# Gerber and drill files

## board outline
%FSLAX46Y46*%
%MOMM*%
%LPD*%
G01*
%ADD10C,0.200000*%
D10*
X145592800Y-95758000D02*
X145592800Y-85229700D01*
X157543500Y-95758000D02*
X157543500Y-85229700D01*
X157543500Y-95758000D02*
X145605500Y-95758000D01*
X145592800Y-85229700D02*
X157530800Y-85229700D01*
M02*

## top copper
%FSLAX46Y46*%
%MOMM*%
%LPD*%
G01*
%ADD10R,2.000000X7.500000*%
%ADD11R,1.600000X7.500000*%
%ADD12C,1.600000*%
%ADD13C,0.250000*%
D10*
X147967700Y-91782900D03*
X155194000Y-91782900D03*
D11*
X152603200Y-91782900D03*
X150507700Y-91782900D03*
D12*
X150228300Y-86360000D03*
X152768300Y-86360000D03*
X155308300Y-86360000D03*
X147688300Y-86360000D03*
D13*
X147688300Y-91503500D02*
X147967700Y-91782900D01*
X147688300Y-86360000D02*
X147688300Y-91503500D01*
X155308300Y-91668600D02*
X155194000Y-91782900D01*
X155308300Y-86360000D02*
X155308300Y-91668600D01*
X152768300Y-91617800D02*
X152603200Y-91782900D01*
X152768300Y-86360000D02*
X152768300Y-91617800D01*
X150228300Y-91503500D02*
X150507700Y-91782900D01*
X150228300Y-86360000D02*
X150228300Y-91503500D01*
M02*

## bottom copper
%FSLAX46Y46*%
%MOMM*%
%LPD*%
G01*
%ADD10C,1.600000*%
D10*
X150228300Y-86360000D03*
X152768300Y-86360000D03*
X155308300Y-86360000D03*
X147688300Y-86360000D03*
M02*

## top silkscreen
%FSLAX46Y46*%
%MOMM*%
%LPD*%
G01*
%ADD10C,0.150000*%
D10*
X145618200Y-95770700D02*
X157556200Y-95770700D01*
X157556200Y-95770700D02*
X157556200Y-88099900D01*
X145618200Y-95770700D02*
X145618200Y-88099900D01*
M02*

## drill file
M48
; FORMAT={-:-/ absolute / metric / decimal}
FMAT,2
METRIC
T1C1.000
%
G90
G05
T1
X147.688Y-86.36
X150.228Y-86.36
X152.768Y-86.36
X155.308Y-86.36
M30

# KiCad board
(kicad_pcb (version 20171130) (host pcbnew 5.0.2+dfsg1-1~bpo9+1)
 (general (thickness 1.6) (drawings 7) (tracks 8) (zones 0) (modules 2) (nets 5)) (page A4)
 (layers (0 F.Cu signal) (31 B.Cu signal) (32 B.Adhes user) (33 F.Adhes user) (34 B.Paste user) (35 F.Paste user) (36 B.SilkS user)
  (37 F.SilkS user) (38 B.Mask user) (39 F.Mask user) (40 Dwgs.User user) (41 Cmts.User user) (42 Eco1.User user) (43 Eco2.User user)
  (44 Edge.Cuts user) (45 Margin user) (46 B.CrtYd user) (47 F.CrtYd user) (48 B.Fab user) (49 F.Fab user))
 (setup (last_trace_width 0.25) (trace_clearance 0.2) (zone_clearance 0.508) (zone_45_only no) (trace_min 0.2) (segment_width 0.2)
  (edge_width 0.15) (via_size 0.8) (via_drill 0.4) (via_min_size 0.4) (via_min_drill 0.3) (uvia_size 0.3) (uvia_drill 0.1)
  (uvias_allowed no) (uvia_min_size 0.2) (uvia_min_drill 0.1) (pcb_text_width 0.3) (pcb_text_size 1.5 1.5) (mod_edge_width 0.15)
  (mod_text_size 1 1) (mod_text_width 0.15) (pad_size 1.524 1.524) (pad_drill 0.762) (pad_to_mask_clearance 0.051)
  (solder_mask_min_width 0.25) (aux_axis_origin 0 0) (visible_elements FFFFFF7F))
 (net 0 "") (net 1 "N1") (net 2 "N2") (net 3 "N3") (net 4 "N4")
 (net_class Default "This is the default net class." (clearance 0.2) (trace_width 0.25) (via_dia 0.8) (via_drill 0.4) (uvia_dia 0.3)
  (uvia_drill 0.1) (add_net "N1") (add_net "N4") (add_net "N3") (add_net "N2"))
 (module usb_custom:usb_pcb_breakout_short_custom (layer F.Cu) (at 151.5237 95.7707)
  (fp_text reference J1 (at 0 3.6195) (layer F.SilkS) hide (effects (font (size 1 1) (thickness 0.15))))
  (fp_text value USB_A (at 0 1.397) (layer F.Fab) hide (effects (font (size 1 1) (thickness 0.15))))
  (fp_line (start -5.9055 0) (end 6.0325 0) (layer F.SilkS) (width 0.15))
  (fp_line (start 6.0325 0) (end 6.0325 -7.6708) (layer F.SilkS) (width 0.15))
  (fp_line (start -5.9055 0) (end -5.9055 -7.6708) (layer F.SilkS) (width 0.15))
  (pad 1 smd rect (at -3.556 -3.9878) (size 2 7.5) (layers F.Cu F.Paste F.Mask) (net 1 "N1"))
  (pad 4 smd rect (at 3.6703 -3.9878) (size 2 7.5) (layers F.Cu F.Paste F.Mask) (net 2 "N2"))
  (pad 3 smd rect (at 1.0795 -3.9878) (size 1.6 7.5) (layers F.Cu F.Paste F.Mask) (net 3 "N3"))
  (pad 2 smd rect (at -1.016 -3.9878) (size 1.6 7.5) (layers F.Cu F.Paste F.Mask) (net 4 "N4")))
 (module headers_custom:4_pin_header (layer F.Cu) (at 151.4983 86.36)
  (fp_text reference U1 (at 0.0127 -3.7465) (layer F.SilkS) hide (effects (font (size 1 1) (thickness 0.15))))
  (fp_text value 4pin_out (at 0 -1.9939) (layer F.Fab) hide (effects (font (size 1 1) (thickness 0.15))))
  (pad 2 thru_hole circle (at -1.27 0) (size 1.6 1.6) (drill 1) (layers *.Cu *.Mask) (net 4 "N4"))
  (pad 3 thru_hole circle (at 1.27 0) (size 1.6 1.6) (drill 1) (layers *.Cu *.Mask) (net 3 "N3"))
  (pad 4 thru_hole circle (at 3.81 0) (size 1.6 1.6) (drill 1) (layers *.Cu *.Mask) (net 2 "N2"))
  (pad 1 thru_hole circle (at -3.81 0) (size 1.6 1.6) (drill 1) (layers *.Cu *.Mask) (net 1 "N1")))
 (gr_line (start 145.5928 95.758) (end 145.5928 85.2297) (layer Edge.Cuts) (width 0.2))
 (gr_line (start 157.5435 95.758) (end 157.5435 85.2297) (layer Edge.Cuts) (width 0.2))
 (gr_line (start 157.5435 95.758) (end 145.6055 95.758) (layer Edge.Cuts) (width 0.2))
 (gr_line (start 145.5928 85.2297) (end 157.5308 85.2297) (layer Edge.Cuts) (width 0.2))
 (segment (start 147.6883 91.5035) (end 147.9677 91.7829) (width 0.25) (layer F.Cu) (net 1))
 (segment (start 147.6883 86.36) (end 147.6883 91.5035) (width 0.25) (layer F.Cu) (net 1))
 (segment (start 155.3083 91.6686) (end 155.194 91.7829) (width 0.25) (layer F.Cu) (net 2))
 (segment (start 155.3083 86.36) (end 155.3083 91.6686) (width 0.25) (layer F.Cu) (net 2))
 (segment (start 152.7683 91.6178) (end 152.6032 91.7829) (width 0.25) (layer F.Cu) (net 3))
 (segment (start 152.7683 86.36) (end 152.7683 91.6178) (width 0.25) (layer F.Cu) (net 3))
 (segment (start 150.2283 91.5035) (end 150.5077 91.7829) (width 0.25) (layer F.Cu) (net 4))
 (segment (start 150.2283 86.36) (end 150.2283 91.5035) (width 0.25) (layer F.Cu) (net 4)))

